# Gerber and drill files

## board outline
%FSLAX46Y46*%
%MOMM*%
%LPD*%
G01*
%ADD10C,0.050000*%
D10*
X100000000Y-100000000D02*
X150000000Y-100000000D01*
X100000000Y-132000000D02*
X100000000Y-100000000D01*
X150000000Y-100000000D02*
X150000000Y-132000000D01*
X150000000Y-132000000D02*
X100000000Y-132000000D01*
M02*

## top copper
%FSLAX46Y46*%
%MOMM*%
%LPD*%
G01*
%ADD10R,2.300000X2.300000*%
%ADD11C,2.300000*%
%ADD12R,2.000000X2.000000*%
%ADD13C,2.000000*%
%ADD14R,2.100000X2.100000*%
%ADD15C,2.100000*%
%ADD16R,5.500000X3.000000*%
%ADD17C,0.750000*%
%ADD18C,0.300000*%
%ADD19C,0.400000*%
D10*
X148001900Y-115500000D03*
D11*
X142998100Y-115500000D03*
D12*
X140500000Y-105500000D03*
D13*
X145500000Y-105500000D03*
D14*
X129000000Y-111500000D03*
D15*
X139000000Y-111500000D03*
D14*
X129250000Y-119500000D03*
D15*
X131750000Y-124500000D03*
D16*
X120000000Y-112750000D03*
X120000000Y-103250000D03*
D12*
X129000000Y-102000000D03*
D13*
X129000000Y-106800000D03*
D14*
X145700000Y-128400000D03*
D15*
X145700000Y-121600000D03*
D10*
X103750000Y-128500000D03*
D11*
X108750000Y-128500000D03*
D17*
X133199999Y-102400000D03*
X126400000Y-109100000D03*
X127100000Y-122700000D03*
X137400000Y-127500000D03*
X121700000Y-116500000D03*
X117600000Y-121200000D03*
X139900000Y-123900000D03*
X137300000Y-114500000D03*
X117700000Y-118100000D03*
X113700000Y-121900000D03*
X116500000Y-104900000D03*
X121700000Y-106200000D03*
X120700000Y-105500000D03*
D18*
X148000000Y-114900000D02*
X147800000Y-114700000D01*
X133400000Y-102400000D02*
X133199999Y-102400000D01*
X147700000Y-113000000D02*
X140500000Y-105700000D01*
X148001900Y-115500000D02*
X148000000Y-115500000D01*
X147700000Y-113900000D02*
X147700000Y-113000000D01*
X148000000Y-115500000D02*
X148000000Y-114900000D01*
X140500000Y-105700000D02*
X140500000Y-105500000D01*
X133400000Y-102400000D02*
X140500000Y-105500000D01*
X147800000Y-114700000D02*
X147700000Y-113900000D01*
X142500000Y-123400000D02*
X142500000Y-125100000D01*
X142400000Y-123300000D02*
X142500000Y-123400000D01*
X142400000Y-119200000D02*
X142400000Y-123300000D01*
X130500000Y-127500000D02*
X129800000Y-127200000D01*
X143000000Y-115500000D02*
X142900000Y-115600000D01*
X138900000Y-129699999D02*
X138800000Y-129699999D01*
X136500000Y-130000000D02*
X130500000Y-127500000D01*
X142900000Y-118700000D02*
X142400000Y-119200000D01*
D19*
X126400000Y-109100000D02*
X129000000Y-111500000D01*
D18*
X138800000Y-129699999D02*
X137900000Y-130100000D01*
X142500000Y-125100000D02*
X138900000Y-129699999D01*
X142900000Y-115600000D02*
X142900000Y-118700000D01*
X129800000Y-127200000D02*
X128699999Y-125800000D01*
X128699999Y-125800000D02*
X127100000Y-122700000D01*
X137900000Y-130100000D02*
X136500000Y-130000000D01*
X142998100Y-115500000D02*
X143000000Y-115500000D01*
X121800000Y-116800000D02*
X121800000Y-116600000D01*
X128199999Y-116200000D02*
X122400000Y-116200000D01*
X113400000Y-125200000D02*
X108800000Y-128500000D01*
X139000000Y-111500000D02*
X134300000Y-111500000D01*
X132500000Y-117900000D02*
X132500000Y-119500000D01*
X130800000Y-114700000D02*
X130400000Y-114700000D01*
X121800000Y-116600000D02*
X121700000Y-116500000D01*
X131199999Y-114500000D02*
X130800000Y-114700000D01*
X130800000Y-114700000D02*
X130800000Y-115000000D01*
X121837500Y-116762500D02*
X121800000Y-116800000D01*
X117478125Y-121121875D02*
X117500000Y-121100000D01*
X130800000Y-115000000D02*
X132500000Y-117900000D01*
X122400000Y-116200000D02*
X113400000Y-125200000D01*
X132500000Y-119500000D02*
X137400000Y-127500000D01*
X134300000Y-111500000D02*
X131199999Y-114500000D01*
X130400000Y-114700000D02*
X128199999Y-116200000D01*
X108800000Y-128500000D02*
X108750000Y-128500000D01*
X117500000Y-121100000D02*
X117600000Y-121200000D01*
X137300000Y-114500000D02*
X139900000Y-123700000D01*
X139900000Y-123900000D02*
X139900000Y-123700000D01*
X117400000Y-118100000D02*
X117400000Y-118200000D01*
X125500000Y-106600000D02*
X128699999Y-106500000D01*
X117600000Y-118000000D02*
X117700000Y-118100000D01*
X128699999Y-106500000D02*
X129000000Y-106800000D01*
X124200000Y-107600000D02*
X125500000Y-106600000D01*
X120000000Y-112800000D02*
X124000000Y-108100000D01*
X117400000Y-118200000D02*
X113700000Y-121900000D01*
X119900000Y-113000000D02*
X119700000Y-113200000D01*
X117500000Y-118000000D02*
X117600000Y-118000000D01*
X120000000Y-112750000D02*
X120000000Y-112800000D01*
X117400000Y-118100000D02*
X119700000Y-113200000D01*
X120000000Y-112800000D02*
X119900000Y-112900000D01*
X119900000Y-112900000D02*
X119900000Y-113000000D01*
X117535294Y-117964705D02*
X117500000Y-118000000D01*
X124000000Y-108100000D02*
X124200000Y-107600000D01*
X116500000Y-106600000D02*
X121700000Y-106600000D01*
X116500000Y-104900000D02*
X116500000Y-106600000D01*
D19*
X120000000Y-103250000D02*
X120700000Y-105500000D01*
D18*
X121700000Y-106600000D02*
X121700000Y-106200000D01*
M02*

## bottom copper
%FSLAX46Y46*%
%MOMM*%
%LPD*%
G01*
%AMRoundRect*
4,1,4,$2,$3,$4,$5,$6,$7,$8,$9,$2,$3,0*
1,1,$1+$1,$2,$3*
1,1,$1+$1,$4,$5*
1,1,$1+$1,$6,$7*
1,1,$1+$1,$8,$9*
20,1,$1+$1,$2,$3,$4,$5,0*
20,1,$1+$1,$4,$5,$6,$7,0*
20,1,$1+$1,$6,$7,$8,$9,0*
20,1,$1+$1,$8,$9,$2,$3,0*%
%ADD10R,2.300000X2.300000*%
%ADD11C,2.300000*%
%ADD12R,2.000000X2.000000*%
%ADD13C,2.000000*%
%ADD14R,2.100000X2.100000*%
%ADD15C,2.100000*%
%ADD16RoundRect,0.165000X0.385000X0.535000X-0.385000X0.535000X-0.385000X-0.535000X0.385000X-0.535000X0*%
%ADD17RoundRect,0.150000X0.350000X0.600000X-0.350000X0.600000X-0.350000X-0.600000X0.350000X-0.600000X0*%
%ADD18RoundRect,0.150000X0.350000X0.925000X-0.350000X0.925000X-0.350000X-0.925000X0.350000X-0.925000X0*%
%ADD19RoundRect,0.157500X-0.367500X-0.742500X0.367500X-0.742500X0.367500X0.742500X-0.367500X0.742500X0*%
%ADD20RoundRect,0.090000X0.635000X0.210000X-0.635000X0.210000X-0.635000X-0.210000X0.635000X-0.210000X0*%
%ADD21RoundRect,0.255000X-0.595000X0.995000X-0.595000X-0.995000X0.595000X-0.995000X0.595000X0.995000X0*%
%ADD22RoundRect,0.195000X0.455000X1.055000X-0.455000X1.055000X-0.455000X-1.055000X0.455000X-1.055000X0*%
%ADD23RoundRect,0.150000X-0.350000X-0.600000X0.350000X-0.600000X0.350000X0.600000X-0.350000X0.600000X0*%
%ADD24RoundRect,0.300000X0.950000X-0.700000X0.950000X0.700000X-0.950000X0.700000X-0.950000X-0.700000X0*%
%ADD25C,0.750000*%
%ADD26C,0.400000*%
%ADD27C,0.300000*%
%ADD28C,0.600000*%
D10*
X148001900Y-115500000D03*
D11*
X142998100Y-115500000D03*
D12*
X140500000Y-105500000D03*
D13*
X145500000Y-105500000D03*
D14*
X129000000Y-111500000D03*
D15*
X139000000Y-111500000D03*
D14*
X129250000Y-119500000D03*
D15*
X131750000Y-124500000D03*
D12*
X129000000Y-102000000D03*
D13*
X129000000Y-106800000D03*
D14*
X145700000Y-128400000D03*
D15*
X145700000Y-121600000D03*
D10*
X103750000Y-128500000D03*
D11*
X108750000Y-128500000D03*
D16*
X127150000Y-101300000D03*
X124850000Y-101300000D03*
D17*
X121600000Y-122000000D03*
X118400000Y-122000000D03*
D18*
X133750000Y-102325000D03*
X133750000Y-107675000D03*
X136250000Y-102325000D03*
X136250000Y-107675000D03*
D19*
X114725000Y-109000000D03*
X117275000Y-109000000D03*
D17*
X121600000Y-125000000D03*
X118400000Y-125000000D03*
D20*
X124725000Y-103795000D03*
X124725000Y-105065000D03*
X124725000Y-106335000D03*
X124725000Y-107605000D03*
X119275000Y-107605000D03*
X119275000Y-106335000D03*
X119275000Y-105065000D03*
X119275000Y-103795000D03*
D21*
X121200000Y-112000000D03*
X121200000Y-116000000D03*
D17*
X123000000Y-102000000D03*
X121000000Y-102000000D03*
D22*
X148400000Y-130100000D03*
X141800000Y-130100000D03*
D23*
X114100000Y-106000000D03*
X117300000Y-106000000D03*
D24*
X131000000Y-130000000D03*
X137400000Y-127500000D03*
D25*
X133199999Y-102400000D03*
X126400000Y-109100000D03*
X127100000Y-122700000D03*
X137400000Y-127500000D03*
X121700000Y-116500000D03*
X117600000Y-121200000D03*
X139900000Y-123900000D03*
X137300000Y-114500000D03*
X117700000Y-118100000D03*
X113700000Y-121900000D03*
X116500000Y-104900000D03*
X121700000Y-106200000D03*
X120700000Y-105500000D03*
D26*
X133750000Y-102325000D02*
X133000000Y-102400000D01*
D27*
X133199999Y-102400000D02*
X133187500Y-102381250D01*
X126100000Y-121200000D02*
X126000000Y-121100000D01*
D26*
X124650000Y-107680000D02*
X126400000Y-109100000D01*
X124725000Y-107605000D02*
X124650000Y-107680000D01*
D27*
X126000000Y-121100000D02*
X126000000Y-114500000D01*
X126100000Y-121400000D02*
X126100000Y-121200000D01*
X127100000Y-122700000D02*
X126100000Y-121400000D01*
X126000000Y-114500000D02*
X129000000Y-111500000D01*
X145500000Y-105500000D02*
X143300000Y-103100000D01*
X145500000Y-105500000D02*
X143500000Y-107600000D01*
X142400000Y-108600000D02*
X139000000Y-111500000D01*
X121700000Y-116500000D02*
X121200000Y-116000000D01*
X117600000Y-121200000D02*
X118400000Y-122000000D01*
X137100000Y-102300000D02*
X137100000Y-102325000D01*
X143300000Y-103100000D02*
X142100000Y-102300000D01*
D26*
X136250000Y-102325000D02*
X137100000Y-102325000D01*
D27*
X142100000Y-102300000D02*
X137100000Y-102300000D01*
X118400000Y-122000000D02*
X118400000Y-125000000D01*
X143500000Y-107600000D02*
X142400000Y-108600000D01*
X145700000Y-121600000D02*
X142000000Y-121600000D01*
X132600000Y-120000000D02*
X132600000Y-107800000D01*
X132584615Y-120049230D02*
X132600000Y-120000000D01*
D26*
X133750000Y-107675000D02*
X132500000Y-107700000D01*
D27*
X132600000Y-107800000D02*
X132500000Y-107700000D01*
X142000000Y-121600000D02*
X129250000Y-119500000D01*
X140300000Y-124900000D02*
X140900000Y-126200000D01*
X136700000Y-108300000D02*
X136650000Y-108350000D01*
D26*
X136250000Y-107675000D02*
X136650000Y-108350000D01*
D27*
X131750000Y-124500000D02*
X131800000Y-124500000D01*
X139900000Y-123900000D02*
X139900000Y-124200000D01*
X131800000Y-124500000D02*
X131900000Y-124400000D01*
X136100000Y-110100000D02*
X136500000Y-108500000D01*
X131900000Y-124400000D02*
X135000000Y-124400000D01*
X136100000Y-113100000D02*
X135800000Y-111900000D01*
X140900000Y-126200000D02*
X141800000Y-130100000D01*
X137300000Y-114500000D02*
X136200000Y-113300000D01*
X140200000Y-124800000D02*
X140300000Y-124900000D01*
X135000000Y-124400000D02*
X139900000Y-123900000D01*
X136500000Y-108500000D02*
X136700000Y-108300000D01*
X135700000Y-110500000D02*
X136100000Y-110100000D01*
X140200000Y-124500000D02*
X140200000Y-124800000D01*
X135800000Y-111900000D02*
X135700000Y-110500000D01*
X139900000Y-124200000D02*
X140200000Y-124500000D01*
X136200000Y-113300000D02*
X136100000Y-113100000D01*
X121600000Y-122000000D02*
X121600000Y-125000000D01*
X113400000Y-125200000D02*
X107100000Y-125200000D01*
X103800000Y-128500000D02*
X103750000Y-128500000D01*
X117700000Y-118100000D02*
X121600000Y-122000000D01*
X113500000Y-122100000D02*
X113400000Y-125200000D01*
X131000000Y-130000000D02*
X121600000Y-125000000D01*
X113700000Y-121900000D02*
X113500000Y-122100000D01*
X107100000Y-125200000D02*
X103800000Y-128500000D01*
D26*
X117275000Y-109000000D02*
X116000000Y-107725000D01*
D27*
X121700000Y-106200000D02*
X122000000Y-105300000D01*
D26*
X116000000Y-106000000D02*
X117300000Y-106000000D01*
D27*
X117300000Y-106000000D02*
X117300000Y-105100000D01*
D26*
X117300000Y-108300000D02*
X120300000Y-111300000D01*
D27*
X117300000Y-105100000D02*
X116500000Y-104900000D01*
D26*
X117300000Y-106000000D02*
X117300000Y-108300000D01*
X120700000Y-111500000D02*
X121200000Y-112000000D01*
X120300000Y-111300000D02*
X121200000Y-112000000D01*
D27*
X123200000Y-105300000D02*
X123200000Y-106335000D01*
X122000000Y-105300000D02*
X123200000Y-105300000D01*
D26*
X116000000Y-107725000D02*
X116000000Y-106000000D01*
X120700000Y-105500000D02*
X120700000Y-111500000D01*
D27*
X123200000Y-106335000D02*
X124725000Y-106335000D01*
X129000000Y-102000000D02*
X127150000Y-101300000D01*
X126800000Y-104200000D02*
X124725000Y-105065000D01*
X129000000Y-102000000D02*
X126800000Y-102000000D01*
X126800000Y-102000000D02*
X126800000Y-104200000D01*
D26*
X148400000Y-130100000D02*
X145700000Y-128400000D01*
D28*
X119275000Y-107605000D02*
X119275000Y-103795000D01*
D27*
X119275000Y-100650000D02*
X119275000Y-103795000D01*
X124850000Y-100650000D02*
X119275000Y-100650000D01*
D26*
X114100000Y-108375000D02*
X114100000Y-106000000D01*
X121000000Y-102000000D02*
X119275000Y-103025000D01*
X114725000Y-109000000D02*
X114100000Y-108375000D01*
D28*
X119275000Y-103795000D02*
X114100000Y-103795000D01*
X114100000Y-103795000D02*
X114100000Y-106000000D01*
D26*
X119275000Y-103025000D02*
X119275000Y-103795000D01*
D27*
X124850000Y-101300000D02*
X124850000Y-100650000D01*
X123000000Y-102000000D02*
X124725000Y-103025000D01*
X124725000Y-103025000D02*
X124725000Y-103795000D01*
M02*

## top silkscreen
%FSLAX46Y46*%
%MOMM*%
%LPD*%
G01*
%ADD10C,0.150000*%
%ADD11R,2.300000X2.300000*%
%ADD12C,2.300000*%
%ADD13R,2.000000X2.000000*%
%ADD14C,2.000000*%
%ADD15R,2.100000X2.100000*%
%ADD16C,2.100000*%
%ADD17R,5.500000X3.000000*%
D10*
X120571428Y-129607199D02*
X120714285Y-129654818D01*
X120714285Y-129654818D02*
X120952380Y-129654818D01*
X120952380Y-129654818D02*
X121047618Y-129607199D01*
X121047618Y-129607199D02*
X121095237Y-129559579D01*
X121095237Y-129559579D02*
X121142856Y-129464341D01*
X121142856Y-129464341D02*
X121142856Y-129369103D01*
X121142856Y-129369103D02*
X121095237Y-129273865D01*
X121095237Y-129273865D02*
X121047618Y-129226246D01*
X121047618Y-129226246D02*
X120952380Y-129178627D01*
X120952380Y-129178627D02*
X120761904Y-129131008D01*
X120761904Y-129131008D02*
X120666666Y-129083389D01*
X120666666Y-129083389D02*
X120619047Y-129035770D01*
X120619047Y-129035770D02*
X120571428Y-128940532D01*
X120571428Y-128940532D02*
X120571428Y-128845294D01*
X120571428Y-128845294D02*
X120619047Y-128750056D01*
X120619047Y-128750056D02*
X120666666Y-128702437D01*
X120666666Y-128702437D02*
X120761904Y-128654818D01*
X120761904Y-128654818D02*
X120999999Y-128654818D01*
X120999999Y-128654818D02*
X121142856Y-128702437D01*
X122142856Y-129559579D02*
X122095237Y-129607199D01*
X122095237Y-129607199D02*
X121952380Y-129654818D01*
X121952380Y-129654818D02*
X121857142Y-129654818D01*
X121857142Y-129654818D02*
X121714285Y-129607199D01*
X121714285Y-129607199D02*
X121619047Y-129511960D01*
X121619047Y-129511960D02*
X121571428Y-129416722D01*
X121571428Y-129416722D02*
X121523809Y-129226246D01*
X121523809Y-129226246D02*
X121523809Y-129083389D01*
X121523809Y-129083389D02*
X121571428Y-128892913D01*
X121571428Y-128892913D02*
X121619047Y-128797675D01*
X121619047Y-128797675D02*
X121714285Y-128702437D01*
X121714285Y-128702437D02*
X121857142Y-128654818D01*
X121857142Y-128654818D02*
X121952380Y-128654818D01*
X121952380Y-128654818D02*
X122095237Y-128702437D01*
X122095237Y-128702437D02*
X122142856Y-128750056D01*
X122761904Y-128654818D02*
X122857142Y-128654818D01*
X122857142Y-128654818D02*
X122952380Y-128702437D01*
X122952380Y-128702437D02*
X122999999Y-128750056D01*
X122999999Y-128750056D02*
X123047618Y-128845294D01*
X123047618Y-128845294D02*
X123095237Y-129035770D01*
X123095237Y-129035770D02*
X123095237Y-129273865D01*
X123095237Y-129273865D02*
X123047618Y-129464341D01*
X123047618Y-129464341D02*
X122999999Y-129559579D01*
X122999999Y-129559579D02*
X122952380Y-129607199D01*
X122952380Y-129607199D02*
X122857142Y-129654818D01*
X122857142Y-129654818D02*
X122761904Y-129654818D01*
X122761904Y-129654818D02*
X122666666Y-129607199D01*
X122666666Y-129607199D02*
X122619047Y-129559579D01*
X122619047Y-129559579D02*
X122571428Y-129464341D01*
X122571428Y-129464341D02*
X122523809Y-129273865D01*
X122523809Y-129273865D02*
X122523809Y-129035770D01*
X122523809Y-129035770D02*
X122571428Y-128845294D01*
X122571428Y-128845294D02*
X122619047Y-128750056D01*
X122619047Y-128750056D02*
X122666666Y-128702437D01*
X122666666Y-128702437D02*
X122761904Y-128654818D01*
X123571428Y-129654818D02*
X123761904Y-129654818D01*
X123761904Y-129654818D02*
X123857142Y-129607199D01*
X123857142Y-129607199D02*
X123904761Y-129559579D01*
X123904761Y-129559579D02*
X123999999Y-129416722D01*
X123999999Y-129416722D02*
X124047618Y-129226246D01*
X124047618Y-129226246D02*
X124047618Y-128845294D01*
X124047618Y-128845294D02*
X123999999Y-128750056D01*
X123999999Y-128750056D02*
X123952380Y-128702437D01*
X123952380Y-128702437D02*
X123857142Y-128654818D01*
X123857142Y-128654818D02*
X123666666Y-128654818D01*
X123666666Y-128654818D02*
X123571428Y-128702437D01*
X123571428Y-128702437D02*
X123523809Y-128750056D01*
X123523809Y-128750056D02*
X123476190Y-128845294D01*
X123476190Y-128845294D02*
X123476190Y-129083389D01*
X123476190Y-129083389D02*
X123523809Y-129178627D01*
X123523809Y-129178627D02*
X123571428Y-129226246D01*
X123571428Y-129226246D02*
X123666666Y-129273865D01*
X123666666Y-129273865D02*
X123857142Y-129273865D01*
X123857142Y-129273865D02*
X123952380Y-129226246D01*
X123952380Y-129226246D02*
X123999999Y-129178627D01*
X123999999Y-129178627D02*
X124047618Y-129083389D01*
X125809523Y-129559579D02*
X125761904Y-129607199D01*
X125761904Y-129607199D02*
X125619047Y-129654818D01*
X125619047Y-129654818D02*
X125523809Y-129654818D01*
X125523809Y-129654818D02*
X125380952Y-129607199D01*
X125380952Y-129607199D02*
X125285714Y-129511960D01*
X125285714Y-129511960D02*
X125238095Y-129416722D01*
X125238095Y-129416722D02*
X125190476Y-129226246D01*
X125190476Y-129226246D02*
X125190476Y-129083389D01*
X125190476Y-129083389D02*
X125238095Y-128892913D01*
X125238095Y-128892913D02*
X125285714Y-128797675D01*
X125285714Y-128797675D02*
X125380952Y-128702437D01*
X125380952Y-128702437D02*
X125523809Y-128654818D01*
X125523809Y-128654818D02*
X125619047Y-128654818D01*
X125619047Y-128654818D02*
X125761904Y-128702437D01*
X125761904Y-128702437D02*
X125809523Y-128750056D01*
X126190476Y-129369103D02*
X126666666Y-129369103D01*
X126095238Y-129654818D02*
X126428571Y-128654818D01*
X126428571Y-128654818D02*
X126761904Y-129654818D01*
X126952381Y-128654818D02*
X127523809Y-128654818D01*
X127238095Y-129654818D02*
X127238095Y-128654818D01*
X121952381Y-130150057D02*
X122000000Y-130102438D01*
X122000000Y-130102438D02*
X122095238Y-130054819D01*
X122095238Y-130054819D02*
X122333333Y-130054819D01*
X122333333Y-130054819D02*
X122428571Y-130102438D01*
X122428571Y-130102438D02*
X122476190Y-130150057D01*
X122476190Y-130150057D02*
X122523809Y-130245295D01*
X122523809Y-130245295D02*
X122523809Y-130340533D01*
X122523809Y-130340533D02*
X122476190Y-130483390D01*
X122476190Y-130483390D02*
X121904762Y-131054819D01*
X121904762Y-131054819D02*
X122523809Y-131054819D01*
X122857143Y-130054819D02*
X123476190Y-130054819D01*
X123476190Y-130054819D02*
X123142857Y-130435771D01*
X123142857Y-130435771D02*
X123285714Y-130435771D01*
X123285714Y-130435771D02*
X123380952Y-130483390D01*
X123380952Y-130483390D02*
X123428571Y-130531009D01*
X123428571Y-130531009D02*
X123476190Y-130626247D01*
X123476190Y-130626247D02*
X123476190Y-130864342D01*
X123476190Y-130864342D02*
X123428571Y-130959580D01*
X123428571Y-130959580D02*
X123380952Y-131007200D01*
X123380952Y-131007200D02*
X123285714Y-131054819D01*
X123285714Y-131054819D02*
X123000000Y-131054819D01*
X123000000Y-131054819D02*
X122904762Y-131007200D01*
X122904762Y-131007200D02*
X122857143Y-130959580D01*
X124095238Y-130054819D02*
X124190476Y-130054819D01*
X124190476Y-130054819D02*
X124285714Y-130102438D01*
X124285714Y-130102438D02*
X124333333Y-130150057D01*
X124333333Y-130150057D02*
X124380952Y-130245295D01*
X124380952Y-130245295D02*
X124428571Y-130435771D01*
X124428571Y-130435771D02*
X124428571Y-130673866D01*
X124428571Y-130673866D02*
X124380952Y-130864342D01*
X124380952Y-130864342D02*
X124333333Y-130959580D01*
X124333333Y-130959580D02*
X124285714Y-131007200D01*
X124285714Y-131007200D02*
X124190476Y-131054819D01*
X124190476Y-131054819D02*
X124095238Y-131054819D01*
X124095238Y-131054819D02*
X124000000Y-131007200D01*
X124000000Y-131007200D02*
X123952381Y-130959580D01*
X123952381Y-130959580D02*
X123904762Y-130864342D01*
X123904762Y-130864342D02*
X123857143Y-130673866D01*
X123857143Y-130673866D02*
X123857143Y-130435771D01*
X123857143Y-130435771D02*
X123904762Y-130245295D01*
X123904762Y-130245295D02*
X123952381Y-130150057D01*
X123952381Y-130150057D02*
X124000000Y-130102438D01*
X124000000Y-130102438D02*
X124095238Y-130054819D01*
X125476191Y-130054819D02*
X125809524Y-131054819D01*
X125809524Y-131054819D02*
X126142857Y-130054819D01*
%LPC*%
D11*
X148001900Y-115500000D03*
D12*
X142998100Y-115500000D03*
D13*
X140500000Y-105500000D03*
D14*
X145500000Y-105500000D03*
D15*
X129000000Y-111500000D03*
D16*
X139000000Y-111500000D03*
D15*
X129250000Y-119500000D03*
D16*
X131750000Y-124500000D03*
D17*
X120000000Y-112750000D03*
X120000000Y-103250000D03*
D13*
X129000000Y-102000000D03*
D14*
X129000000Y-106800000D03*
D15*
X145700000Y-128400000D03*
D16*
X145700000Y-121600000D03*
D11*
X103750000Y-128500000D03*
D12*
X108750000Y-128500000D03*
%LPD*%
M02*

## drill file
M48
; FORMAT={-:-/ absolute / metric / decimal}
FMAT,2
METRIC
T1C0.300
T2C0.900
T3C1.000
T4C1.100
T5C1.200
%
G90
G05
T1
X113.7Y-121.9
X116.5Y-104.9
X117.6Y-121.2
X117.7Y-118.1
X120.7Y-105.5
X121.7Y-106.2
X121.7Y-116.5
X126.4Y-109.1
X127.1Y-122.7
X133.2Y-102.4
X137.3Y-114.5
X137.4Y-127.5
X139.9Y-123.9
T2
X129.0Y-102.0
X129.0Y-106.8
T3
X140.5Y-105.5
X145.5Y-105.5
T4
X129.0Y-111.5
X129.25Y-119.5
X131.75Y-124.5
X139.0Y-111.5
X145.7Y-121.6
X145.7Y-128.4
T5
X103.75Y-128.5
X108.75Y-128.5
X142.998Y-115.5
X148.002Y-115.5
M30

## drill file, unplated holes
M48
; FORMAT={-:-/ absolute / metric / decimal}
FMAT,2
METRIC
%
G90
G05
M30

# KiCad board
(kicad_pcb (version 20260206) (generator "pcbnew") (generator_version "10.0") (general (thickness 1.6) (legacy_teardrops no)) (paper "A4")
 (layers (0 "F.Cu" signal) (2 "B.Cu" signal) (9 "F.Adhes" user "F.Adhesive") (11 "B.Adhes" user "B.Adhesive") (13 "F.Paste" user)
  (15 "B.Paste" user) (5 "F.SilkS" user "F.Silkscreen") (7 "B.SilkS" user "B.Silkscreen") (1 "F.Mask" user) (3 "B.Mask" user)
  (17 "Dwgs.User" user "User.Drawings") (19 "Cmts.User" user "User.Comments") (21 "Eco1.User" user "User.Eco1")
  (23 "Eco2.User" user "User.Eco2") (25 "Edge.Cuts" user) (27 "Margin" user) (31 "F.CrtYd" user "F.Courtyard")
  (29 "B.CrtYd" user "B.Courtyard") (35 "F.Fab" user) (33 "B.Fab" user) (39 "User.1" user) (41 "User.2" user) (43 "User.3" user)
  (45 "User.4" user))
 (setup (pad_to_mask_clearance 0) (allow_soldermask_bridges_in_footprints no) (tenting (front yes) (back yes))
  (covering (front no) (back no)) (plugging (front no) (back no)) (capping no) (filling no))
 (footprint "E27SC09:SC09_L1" (layer "F.Cu") (at 145.5 115.5 180)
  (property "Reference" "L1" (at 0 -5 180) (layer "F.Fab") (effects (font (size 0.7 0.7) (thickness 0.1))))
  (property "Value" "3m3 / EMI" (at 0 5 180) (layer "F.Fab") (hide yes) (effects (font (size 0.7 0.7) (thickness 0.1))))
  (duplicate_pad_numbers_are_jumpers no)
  (pad "1" thru_hole rect (at -2.5019 0 180) (size 2.3 2.3) (drill 1.2) (layers "*.Cu" "*.Mask") (remove_unused_layers no) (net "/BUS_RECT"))
  (pad "2" thru_hole circle (at 2.5019 0 180) (size 2.3 2.3) (drill 1.2) (layers "*.Cu" "*.Mask") (remove_unused_layers no)
   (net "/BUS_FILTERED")))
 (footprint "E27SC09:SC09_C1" (layer "F.Cu") (at 143 105.5)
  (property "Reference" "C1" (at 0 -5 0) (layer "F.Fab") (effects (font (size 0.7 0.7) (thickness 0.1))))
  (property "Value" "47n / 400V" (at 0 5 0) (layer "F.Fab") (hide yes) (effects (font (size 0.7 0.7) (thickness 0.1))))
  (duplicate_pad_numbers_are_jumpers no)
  (pad "1" thru_hole rect (at -2.5 0) (size 2 2) (drill 1) (layers "*.Cu" "*.Mask") (remove_unused_layers no) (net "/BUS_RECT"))
  (pad "2" thru_hole circle (at 2.5 0) (size 2 2) (drill 1) (layers "*.Cu" "*.Mask") (remove_unused_layers no) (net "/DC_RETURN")))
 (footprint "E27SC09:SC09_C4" (layer "F.Cu") (at 134 111.5)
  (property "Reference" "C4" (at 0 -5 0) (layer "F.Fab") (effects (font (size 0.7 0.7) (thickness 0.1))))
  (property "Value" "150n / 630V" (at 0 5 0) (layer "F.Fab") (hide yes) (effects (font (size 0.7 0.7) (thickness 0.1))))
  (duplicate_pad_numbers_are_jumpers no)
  (pad "1" thru_hole rect (at -5 0) (size 2.1 2.1) (drill 1.1) (layers "*.Cu" "*.Mask") (remove_unused_layers no) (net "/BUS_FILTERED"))
  (pad "2" thru_hole circle (at 5 0) (size 2.1 2.1) (drill 1.1) (layers "*.Cu" "*.Mask") (remove_unused_layers no) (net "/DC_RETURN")))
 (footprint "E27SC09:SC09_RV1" (layer "F.Cu") (at 130.5 122)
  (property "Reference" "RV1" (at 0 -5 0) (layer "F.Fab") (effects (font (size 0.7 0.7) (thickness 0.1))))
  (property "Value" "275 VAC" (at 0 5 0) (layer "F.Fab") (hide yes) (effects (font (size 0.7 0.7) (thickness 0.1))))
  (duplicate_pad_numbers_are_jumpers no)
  (pad "1" thru_hole rect (at -1.25 -2.5) (size 2.1 2.1) (drill 1.1) (layers "*.Cu" "*.Mask") (remove_unused_layers no) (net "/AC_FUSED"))
  (pad "2" thru_hole circle (at 1.25 2.5) (size 2.1 2.1) (drill 1.1) (layers "*.Cu" "*.Mask") (remove_unused_layers no) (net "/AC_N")))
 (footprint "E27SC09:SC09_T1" (layer "F.Cu") (at 120 108)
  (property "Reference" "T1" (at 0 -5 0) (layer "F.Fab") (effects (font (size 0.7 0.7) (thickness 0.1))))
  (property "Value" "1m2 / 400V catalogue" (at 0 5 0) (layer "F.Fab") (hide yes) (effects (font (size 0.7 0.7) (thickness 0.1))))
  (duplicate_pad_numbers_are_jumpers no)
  (pad "1" smd rect (at 0 4.75) (size 5.5 3) (layers "F.Cu" "F.Mask" "F.Paste") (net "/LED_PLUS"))
  (pad "2" smd rect (at 0 -4.75) (size 5.5 3) (layers "F.Cu" "F.Mask" "F.Paste") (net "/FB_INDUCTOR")))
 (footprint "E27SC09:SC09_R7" (layer "F.Cu") (at 129 102)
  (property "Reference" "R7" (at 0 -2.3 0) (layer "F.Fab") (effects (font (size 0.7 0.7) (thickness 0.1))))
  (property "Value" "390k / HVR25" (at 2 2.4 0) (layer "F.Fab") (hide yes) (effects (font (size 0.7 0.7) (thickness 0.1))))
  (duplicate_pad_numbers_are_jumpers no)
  (pad "1" thru_hole rect (at 0 0) (size 2 2) (drill 0.9) (layers "*.Cu" "*.Mask") (remove_unused_layers no) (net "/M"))
  (pad "2" thru_hole circle (at 0 4.8) (size 2 2) (drill 0.9) (layers "*.Cu" "*.Mask") (remove_unused_layers no) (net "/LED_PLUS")))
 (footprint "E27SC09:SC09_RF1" (layer "F.Cu") (at 145.7 128.4 180)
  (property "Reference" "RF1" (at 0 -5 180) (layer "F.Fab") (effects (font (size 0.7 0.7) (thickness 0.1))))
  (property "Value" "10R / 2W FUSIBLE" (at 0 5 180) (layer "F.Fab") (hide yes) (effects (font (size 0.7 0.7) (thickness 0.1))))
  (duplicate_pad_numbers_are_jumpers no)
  (pad "1" thru_hole rect (at 0 0 180) (size 2.1 2.1) (drill 1.1) (layers "*.Cu" "*.Mask") (remove_unused_layers no) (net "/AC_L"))
  (pad "2" thru_hole circle (at 0 6.8 180) (size 2.1 2.1) (drill 1.1) (layers "*.Cu" "*.Mask") (remove_unused_layers no) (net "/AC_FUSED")))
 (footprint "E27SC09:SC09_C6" (layer "F.Cu") (at 106.25 128.5 90)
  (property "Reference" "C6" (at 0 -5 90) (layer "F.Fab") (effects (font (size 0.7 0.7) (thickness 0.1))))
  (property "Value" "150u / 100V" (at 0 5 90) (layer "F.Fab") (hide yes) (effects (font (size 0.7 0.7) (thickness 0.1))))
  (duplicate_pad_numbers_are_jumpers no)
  (pad "1" thru_hole rect (at 0 -2.5 90) (size 2.3 2.3) (drill 1.2) (layers "*.Cu" "*.Mask") (remove_unused_layers no) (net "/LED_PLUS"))
  (pad "2" thru_hole circle (at 0 2.5 90) (size 2.3 2.3) (drill 1.2) (layers "*.Cu" "*.Mask") (remove_unused_layers no) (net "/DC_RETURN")))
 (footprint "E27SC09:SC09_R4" (layer "B.Cu") (at 126 101.3 180)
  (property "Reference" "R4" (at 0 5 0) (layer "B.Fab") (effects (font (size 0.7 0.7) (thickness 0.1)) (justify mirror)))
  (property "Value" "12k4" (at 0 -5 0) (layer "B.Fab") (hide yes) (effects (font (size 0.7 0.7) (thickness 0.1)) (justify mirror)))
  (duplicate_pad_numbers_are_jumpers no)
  (pad "1" smd roundrect (at -1.15 0 180) (size 1.1 1.4) (layers "B.Cu" "B.Mask" "B.Paste") (roundrect_rratio 0.15) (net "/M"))
  (pad "2" smd roundrect (at 1.15 0 180) (size 1.1 1.4) (layers "B.Cu" "B.Mask" "B.Paste") (roundrect_rratio 0.15) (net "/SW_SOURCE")))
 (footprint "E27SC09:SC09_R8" (layer "B.Cu") (at 120 122 180)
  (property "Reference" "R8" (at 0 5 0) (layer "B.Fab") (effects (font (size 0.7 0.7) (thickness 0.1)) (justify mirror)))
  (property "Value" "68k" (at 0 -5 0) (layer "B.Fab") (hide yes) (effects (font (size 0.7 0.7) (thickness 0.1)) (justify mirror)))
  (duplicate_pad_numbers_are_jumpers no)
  (pad "1" smd roundrect (at -1.6 0 180) (size 1 1.5) (layers "B.Cu" "B.Mask" "B.Paste") (roundrect_rratio 0.15) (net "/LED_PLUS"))
  (pad "2" smd roundrect (at 1.6 0 180) (size 1 1.5) (layers "B.Cu" "B.Mask" "B.Paste") (roundrect_rratio 0.15) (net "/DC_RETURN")))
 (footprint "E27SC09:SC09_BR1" (layer "B.Cu") (at 135 105 180)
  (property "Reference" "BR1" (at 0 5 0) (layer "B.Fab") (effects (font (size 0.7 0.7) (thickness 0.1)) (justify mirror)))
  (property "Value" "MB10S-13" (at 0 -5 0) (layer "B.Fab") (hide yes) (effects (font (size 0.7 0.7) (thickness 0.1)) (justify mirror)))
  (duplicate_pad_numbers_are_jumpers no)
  (pad "1" smd roundrect (at 1.25 2.675 180) (size 1 2.15) (layers "B.Cu" "B.Mask" "B.Paste") (roundrect_rratio 0.15) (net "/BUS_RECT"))
  (pad "2" smd roundrect (at 1.25 -2.675 180) (size 1 2.15) (layers "B.Cu" "B.Mask" "B.Paste") (roundrect_rratio 0.15) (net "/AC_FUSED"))
  (pad "3" smd roundrect (at -1.25 2.675 180) (size 1 2.15) (layers "B.Cu" "B.Mask" "B.Paste") (roundrect_rratio 0.15) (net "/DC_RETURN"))
  (pad "4" smd roundrect (at -1.25 -2.675 180) (size 1 2.15) (layers "B.Cu" "B.Mask" "B.Paste") (roundrect_rratio 0.15) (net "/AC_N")))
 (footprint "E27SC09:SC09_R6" (layer "B.Cu") (at 116 109)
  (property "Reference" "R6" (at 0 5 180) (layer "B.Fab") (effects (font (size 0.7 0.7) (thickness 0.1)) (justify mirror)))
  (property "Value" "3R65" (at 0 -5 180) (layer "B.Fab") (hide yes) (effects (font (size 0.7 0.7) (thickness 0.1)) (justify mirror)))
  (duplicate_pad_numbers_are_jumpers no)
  (pad "1" smd roundrect (at -1.275 0) (size 1.05 1.8) (layers "B.Cu" "B.Mask" "B.Paste") (roundrect_rratio 0.15) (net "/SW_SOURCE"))
  (pad "2" smd roundrect (at 1.275 0) (size 1.05 1.8) (layers "B.Cu" "B.Mask" "B.Paste") (roundrect_rratio 0.15) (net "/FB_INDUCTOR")))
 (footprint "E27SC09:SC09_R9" (layer "B.Cu") (at 120 125 180)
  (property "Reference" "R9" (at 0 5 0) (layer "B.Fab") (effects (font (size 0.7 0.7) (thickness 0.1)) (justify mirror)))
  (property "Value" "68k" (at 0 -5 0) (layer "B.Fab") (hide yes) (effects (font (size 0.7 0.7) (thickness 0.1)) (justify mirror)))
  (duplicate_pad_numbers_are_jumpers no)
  (pad "1" smd roundrect (at -1.6 0 180) (size 1 1.5) (layers "B.Cu" "B.Mask" "B.Paste") (roundrect_rratio 0.15) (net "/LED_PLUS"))
  (pad "2" smd roundrect (at 1.6 0 180) (size 1 1.5) (layers "B.Cu" "B.Mask" "B.Paste") (roundrect_rratio 0.15) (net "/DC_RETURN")))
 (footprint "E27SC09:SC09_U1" (layer "B.Cu") (at 122 105.7 180)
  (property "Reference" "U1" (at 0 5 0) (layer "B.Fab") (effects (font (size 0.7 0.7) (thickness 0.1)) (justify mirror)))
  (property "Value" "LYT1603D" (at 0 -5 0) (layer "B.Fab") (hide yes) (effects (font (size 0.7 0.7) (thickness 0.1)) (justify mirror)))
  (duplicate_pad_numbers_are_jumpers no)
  (pad "1" smd roundrect (at -2.725 1.905 180) (size 1.45 0.6) (layers "B.Cu" "B.Mask" "B.Paste") (roundrect_rratio 0.15) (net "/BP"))
  (pad "2" smd roundrect (at -2.725 0.635 180) (size 1.45 0.6) (layers "B.Cu" "B.Mask" "B.Paste") (roundrect_rratio 0.15) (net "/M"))
  (pad "3" smd roundrect (at -2.725 -0.635 180) (size 1.45 0.6) (layers "B.Cu" "B.Mask" "B.Paste") (roundrect_rratio 0.15)
   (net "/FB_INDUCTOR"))
  (pad "4" smd roundrect (at -2.725 -1.905 180) (size 1.45 0.6) (layers "B.Cu" "B.Mask" "B.Paste") (roundrect_rratio 0.15)
   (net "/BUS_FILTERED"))
  (pad "5" smd roundrect (at 2.725 -1.905 180) (size 1.45 0.6) (layers "B.Cu" "B.Mask" "B.Paste") (roundrect_rratio 0.15) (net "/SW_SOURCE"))
  (pad "6" smd roundrect (at 2.725 -0.635 180) (size 1.45 0.6) (layers "B.Cu" "B.Mask" "B.Paste") (roundrect_rratio 0.15) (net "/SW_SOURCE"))
  (pad "7" smd roundrect (at 2.725 0.635 180) (size 1.45 0.6) (layers "B.Cu" "B.Mask" "B.Paste") (roundrect_rratio 0.15) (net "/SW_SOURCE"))
  (pad "8" smd roundrect (at 2.725 1.905 180) (size 1.45 0.6) (layers "B.Cu" "B.Mask" "B.Paste") (roundrect_rratio 0.15) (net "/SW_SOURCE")))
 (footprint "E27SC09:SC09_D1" (layer "B.Cu") (at 121.2 114 -90)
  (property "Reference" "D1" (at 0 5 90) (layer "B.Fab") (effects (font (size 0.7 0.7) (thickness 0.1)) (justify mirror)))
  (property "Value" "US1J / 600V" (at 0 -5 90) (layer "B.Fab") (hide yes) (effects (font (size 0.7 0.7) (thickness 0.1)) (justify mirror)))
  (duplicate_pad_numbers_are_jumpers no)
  (pad "1" smd roundrect (at -2 0 270) (size 2.5 1.7) (layers "B.Cu" "B.Mask" "B.Paste") (roundrect_rratio 0.15) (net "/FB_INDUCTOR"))
  (pad "2" smd roundrect (at 2 0 270) (size 2.5 1.7) (layers "B.Cu" "B.Mask" "B.Paste") (roundrect_rratio 0.15) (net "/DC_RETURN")))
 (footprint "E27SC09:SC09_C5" (layer "B.Cu") (at 122 102 180)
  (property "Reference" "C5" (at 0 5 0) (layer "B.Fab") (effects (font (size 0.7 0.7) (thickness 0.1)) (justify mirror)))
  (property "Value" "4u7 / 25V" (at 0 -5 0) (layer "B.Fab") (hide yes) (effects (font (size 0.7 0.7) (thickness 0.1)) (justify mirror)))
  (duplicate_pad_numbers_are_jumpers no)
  (pad "1" smd roundrect (at -1 0 180) (size 1 1.5) (layers "B.Cu" "B.Mask" "B.Paste") (roundrect_rratio 0.15) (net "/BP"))
  (pad "2" smd roundrect (at 1 0 180) (size 1 1.5) (layers "B.Cu" "B.Mask" "B.Paste") (roundrect_rratio 0.15) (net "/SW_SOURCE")))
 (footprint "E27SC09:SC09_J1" (layer "B.Cu") (at 148.4 130.1 180)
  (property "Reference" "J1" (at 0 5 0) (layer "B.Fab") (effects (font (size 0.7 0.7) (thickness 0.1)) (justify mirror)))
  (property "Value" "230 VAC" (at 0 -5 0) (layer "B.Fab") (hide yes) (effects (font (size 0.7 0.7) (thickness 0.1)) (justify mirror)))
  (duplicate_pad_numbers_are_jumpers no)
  (pad "1" smd roundrect (at 0 0 180) (size 1.3 2.5) (layers "B.Cu" "B.Mask" "B.Paste") (roundrect_rratio 0.15) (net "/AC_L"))
  (pad "2" smd roundrect (at 6.6 0 180) (size 1.3 2.5) (layers "B.Cu" "B.Mask" "B.Paste") (roundrect_rratio 0.15) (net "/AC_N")))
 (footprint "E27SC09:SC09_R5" (layer "B.Cu") (at 115.7 106)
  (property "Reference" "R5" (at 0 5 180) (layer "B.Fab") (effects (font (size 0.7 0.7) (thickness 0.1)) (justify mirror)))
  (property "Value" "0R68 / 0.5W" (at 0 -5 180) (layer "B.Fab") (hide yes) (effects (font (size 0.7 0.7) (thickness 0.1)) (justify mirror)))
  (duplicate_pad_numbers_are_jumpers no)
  (pad "1" smd roundrect (at -1.6 0) (size 1 1.5) (layers "B.Cu" "B.Mask" "B.Paste") (roundrect_rratio 0.15) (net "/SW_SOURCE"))
  (pad "2" smd roundrect (at 1.6 0) (size 1 1.5) (layers "B.Cu" "B.Mask" "B.Paste") (roundrect_rratio 0.15) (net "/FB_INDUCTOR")))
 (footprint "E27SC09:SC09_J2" (layer "B.Cu") (at 131 130 90)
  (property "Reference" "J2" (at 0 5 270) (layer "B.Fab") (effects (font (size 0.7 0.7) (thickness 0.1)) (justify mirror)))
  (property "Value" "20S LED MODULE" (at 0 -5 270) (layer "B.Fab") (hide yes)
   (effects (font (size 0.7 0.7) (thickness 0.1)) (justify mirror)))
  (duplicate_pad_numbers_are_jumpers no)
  (pad "1" smd roundrect (at 0 0 90) (size 2 2.5) (layers "B.Cu" "B.Mask" "B.Paste") (roundrect_rratio 0.15) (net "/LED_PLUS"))
  (pad "2" smd roundrect (at 2.5 6.4 90) (size 2 2.5) (layers "B.Cu" "B.Mask" "B.Paste") (roundrect_rratio 0.15) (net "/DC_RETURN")))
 (gr_line (start 100 100) (end 150 100) (stroke (width 0.05) (type default)) (layer "Edge.Cuts"))
 (gr_line (start 100 132) (end 100 100) (stroke (width 0.05) (type default)) (layer "Edge.Cuts"))
 (gr_line (start 150 100) (end 150 132) (stroke (width 0.05) (type default)) (layer "Edge.Cuts"))
 (gr_line (start 150 132) (end 100 132) (stroke (width 0.05) (type default)) (layer "Edge.Cuts"))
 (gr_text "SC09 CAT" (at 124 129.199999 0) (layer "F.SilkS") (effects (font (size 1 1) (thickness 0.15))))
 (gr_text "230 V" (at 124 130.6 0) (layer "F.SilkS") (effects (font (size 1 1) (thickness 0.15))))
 (segment (start 148 114.9) (end 147.8 114.7) (width 0.3) (layer "F.Cu") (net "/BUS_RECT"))
 (segment (start 133.4 102.4) (end 133.199999 102.4) (width 0.3) (layer "F.Cu") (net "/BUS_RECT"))
 (segment (start 147.7 113) (end 140.5 105.7) (width 0.3) (layer "F.Cu") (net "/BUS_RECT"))
 (segment (start 148.0019 115.5) (end 148 115.5) (width 0.3) (layer "F.Cu") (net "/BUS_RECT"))
 (segment (start 147.7 113.9) (end 147.7 113) (width 0.3) (layer "F.Cu") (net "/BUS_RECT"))
 (segment (start 148 115.5) (end 148 114.9) (width 0.3) (layer "F.Cu") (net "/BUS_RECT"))
 (segment (start 140.5 105.7) (end 140.5 105.5) (width 0.3) (layer "F.Cu") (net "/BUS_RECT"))
 (segment (start 133.4 102.4) (end 140.5 105.5) (width 0.3) (layer "F.Cu") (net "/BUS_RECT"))
 (segment (start 147.8 114.7) (end 147.7 113.9) (width 0.3) (layer "F.Cu") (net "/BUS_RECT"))
 (via (at 133.199999 102.4) (size 0.75) (drill 0.3) (layers "F.Cu" "B.Cu") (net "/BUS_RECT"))
 (segment (start 133.75 102.325) (end 133 102.4) (width 0.4) (layer "B.Cu") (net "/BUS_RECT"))
 (segment (start 133.199999 102.4) (end 133.1875 102.38125) (width 0.3) (layer "B.Cu") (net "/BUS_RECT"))
 (segment (start 142.5 123.4) (end 142.5 125.1) (width 0.3) (layer "F.Cu") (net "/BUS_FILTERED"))
 (segment (start 142.4 123.3) (end 142.5 123.4) (width 0.3) (layer "F.Cu") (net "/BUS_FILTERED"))
 (segment (start 142.4 119.2) (end 142.4 123.3) (width 0.3) (layer "F.Cu") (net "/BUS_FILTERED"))
 (segment (start 130.5 127.5) (end 129.8 127.2) (width 0.3) (layer "F.Cu") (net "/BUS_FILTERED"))
 (segment (start 143 115.5) (end 142.9 115.6) (width 0.3) (layer "F.Cu") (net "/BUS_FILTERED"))
 (segment (start 138.9 129.699999) (end 138.8 129.699999) (width 0.3) (layer "F.Cu") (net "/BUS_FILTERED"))
 (segment (start 136.5 130) (end 130.5 127.5) (width 0.3) (layer "F.Cu") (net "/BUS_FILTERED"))
 (segment (start 142.9 118.7) (end 142.4 119.2) (width 0.3) (layer "F.Cu") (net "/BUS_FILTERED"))
 (segment (start 126.4 109.1) (end 129 111.5) (width 0.4) (layer "F.Cu") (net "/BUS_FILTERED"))
 (segment (start 138.8 129.699999) (end 137.9 130.1) (width 0.3) (layer "F.Cu") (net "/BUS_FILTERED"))
 (segment (start 142.5 125.1) (end 138.9 129.699999) (width 0.3) (layer "F.Cu") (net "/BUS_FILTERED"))
 (segment (start 142.9 115.6) (end 142.9 118.7) (width 0.3) (layer "F.Cu") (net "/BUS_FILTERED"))
 (segment (start 129.8 127.2) (end 128.699999 125.8) (width 0.3) (layer "F.Cu") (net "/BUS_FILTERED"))
 (segment (start 128.699999 125.8) (end 127.1 122.7) (width 0.3) (layer "F.Cu") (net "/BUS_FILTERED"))
 (segment (start 137.9 130.1) (end 136.5 130) (width 0.3) (layer "F.Cu") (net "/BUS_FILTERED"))
 (segment (start 142.9981 115.5) (end 143 115.5) (width 0.3) (layer "F.Cu") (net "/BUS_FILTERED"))
 (via (at 126.4 109.1) (size 0.75) (drill 0.3) (layers "F.Cu" "B.Cu") (tenting (front yes) (back yes)) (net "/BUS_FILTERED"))
 (via (at 127.1 122.7) (size 0.75) (drill 0.3) (layers "F.Cu" "B.Cu") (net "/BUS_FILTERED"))
 (segment (start 126.1 121.2) (end 126 121.1) (width 0.3) (layer "B.Cu") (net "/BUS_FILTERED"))
 (segment (start 124.65 107.68) (end 126.4 109.1) (width 0.4) (layer "B.Cu") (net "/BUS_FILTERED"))
 (segment (start 124.725 107.605) (end 124.65 107.68) (width 0.4) (layer "B.Cu") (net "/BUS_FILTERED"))
 (segment (start 126 121.1) (end 126 114.5) (width 0.3) (layer "B.Cu") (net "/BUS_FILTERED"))
 (segment (start 126.1 121.4) (end 126.1 121.2) (width 0.3) (layer "B.Cu") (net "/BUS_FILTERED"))
 (segment (start 127.1 122.7) (end 126.1 121.4) (width 0.3) (layer "B.Cu") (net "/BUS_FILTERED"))
 (segment (start 126 114.5) (end 129 111.5) (width 0.3) (layer "B.Cu") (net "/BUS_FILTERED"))
 (segment (start 121.8 116.8) (end 121.8 116.6) (width 0.3) (layer "F.Cu") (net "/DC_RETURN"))
 (segment (start 128.199999 116.2) (end 122.4 116.2) (width 0.3) (layer "F.Cu") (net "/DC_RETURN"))
 (segment (start 113.4 125.2) (end 108.8 128.5) (width 0.3) (layer "F.Cu") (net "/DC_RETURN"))
 (segment (start 139 111.5) (end 134.3 111.5) (width 0.3) (layer "F.Cu") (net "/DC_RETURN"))
 (segment (start 132.5 117.9) (end 132.5 119.5) (width 0.3) (layer "F.Cu") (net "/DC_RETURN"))
 (segment (start 130.8 114.7) (end 130.4 114.7) (width 0.3) (layer "F.Cu") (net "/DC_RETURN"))
 (segment (start 121.8 116.6) (end 121.7 116.5) (width 0.3) (layer "F.Cu") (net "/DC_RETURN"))
 (segment (start 131.199999 114.5) (end 130.8 114.7) (width 0.3) (layer "F.Cu") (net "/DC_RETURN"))
 (segment (start 130.8 114.7) (end 130.8 115) (width 0.3) (layer "F.Cu") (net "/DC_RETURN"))
 (segment (start 121.8375 116.7625) (end 121.8 116.8) (width 0.3) (layer "F.Cu") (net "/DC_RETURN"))
 (segment (start 117.478125 121.121875) (end 117.5 121.1) (width 0.3) (layer "F.Cu") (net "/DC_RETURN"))
 (segment (start 130.8 115) (end 132.5 117.9) (width 0.3) (layer "F.Cu") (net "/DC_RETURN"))
 (segment (start 122.4 116.2) (end 113.4 125.2) (width 0.3) (layer "F.Cu") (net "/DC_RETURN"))
 (segment (start 132.5 119.5) (end 137.4 127.5) (width 0.3) (layer "F.Cu") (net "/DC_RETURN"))
 (segment (start 134.3 111.5) (end 131.199999 114.5) (width 0.3) (layer "F.Cu") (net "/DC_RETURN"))
 (segment (start 130.4 114.7) (end 128.199999 116.2) (width 0.3) (layer "F.Cu") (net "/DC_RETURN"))
 (segment (start 108.8 128.5) (end 108.75 128.5) (width 0.3) (layer "F.Cu") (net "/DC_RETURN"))
 (segment (start 117.5 121.1) (end 117.6 121.2) (width 0.3) (layer "F.Cu") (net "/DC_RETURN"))
 (via (at 137.4 127.5) (size 0.75) (drill 0.3) (layers "F.Cu" "B.Cu") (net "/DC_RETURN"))
 (via (at 121.7 116.5) (size 0.75) (drill 0.3) (layers "F.Cu" "B.Cu") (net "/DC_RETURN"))
 (via (at 117.6 121.2) (size 0.75) (drill 0.3) (layers "F.Cu" "B.Cu") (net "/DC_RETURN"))
 (segment (start 145.5 105.5) (end 143.3 103.1) (width 0.3) (layer "B.Cu") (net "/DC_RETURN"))
 (segment (start 145.5 105.5) (end 143.5 107.6) (width 0.3) (layer "B.Cu") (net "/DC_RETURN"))
 (segment (start 142.4 108.6) (end 139 111.5) (width 0.3) (layer "B.Cu") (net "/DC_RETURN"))
 (segment (start 121.7 116.5) (end 121.2 116) (width 0.3) (layer "B.Cu") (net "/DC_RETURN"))
 (segment (start 117.6 121.2) (end 118.4 122) (width 0.3) (layer "B.Cu") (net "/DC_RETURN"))
 (segment (start 137.1 102.3) (end 137.1 102.325) (width 0.3) (layer "B.Cu") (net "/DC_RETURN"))
 (segment (start 143.3 103.1) (end 142.1 102.3) (width 0.3) (layer "B.Cu") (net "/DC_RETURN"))
 (segment (start 136.25 102.325) (end 137.1 102.325) (width 0.4) (layer "B.Cu") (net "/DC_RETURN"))
 (segment (start 142.1 102.3) (end 137.1 102.3) (width 0.3) (layer "B.Cu") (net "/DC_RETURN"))
 (segment (start 118.4 122) (end 118.4 125) (width 0.3) (layer "B.Cu") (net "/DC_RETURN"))
 (segment (start 143.5 107.6) (end 142.4 108.6) (width 0.3) (layer "B.Cu") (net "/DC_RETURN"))
 (segment (start 145.7 121.6) (end 142 121.6) (width 0.3) (layer "B.Cu") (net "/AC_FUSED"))
 (segment (start 132.6 120) (end 132.6 107.8) (width 0.3) (layer "B.Cu") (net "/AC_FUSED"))
 (segment (start 132.584615 120.04923) (end 132.6 120) (width 0.3) (layer "B.Cu") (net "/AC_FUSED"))
 (segment (start 133.75 107.675) (end 132.5 107.7) (width 0.4) (layer "B.Cu") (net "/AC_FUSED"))
 (segment (start 132.6 107.8) (end 132.5 107.7) (width 0.3) (layer "B.Cu") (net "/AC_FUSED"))
 (segment (start 142 121.6) (end 129.25 119.5) (width 0.3) (layer "B.Cu") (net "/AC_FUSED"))
 (segment (start 137.3 114.5) (end 139.9 123.7) (width 0.3) (layer "F.Cu") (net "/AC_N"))
 (segment (start 139.9 123.9) (end 139.9 123.7) (width 0.3) (layer "F.Cu") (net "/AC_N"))
 (via (at 139.9 123.9) (size 0.75) (drill 0.3) (layers "F.Cu" "B.Cu") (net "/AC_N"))
 (via (at 137.3 114.5) (size 0.75) (drill 0.3) (layers "F.Cu" "B.Cu") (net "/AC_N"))
 (segment (start 140.3 124.9) (end 140.9 126.2) (width 0.3) (layer "B.Cu") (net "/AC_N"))
 (segment (start 136.7 108.3) (end 136.65 108.35) (width 0.3) (layer "B.Cu") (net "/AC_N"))
 (segment (start 136.25 107.675) (end 136.65 108.35) (width 0.4) (layer "B.Cu") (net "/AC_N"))
 (segment (start 131.75 124.5) (end 131.8 124.5) (width 0.3) (layer "B.Cu") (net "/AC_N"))
 (segment (start 139.9 123.9) (end 139.9 124.2) (width 0.3) (layer "B.Cu") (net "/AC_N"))
 (segment (start 131.8 124.5) (end 131.9 124.4) (width 0.3) (layer "B.Cu") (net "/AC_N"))
 (segment (start 136.1 110.1) (end 136.5 108.5) (width 0.3) (layer "B.Cu") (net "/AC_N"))
 (segment (start 131.9 124.4) (end 135 124.4) (width 0.3) (layer "B.Cu") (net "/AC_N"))
 (segment (start 136.1 113.1) (end 135.8 111.9) (width 0.3) (layer "B.Cu") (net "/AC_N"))
 (segment (start 140.9 126.2) (end 141.8 130.1) (width 0.3) (layer "B.Cu") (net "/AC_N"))
 (segment (start 137.3 114.5) (end 136.2 113.3) (width 0.3) (layer "B.Cu") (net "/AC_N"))
 (segment (start 140.2 124.8) (end 140.3 124.9) (width 0.3) (layer "B.Cu") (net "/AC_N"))
 (segment (start 135 124.4) (end 139.9 123.9) (width 0.3) (layer "B.Cu") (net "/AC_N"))
 (segment (start 136.5 108.5) (end 136.7 108.3) (width 0.3) (layer "B.Cu") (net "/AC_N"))
 (segment (start 135.7 110.5) (end 136.1 110.1) (width 0.3) (layer "B.Cu") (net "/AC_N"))
 (segment (start 140.2 124.5) (end 140.2 124.8) (width 0.3) (layer "B.Cu") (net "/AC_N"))
 (segment (start 135.8 111.9) (end 135.7 110.5) (width 0.3) (layer "B.Cu") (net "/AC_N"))
 (segment (start 139.9 124.2) (end 140.2 124.5) (width 0.3) (layer "B.Cu") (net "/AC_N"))
 (segment (start 136.2 113.3) (end 136.1 113.1) (width 0.3) (layer "B.Cu") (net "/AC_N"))
 (segment (start 117.4 118.1) (end 117.4 118.2) (width 0.3) (layer "F.Cu") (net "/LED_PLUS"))
 (segment (start 125.5 106.6) (end 128.699999 106.5) (width 0.3) (layer "F.Cu") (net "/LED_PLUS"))
 (segment (start 117.6 118) (end 117.7 118.1) (width 0.3) (layer "F.Cu") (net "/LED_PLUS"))
 (segment (start 128.699999 106.5) (end 129 106.8) (width 0.3) (layer "F.Cu") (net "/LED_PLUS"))
 (segment (start 124.2 107.6) (end 125.5 106.6) (width 0.3) (layer "F.Cu") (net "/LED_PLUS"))
 (segment (start 120 112.8) (end 124 108.1) (width 0.3) (layer "F.Cu") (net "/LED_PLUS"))
 (segment (start 117.4 118.2) (end 113.7 121.9) (width 0.3) (layer "F.Cu") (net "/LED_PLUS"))
 (segment (start 119.9 113) (end 119.7 113.2) (width 0.3) (layer "F.Cu") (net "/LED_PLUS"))
 (segment (start 117.5 118) (end 117.6 118) (width 0.3) (layer "F.Cu") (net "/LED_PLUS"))
 (segment (start 120 112.75) (end 120 112.8) (width 0.3) (layer "F.Cu") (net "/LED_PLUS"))
 (segment (start 117.4 118.1) (end 119.7 113.2) (width 0.3) (layer "F.Cu") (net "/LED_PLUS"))
 (segment (start 120 112.8) (end 119.9 112.9) (width 0.3) (layer "F.Cu") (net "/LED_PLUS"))
 (segment (start 119.9 112.9) (end 119.9 113) (width 0.3) (layer "F.Cu") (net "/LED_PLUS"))
 (segment (start 117.535294 117.964705) (end 117.5 118) (width 0.3) (layer "F.Cu") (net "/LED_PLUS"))
 (segment (start 124 108.1) (end 124.2 107.6) (width 0.3) (layer "F.Cu") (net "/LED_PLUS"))
 (via (at 117.7 118.1) (size 0.75) (drill 0.3) (layers "F.Cu" "B.Cu") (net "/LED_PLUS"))
 (via (at 113.7 121.9) (size 0.75) (drill 0.3) (layers "F.Cu" "B.Cu") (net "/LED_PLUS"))
 (segment (start 121.6 122) (end 121.6 125) (width 0.3) (layer "B.Cu") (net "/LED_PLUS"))
 (segment (start 113.4 125.2) (end 107.1 125.2) (width 0.3) (layer "B.Cu") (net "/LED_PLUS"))
 (segment (start 103.8 128.5) (end 103.75 128.5) (width 0.3) (layer "B.Cu") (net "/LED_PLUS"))
 (segment (start 117.7 118.1) (end 121.6 122) (width 0.3) (layer "B.Cu") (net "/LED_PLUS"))
 (segment (start 113.5 122.1) (end 113.4 125.2) (width 0.3) (layer "B.Cu") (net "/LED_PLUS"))
 (segment (start 131 130) (end 121.6 125) (width 0.3) (layer "B.Cu") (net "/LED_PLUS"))
 (segment (start 113.7 121.9) (end 113.5 122.1) (width 0.3) (layer "B.Cu") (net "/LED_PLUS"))
 (segment (start 107.1 125.2) (end 103.8 128.5) (width 0.3) (layer "B.Cu") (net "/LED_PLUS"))
 (segment (start 116.5 106.6) (end 121.7 106.6) (width 0.3) (layer "F.Cu") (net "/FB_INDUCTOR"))
 (segment (start 116.5 104.9) (end 116.5 106.6) (width 0.3) (layer "F.Cu") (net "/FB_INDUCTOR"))
 (segment (start 120 103.25) (end 120.7 105.5) (width 0.4) (layer "F.Cu") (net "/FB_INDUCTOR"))
 (segment (start 121.7 106.6) (end 121.7 106.2) (width 0.3) (layer "F.Cu") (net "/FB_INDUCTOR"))
 (via (at 116.5 104.9) (size 0.75) (drill 0.3) (layers "F.Cu" "B.Cu") (tenting (front yes) (back yes)) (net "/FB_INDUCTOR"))
 (via (at 121.7 106.2) (size 0.75) (drill 0.3) (layers "F.Cu" "B.Cu") (tenting (front yes) (back yes)) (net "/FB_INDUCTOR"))
 (via (at 120.7 105.5) (size 0.75) (drill 0.3) (layers "F.Cu" "B.Cu") (tenting (front yes) (back yes)) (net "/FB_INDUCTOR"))
 (segment (start 117.275 109) (end 116 107.725) (width 0.4) (layer "B.Cu") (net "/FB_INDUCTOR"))
 (segment (start 121.7 106.2) (end 122 105.3) (width 0.3) (layer "B.Cu") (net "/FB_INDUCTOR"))
 (segment (start 116 106) (end 117.3 106) (width 0.4) (layer "B.Cu") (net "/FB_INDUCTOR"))
 (segment (start 117.3 106) (end 117.3 105.1) (width 0.3) (layer "B.Cu") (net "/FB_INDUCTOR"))
 (segment (start 117.3 108.3) (end 120.3 111.3) (width 0.4) (layer "B.Cu") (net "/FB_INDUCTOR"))
 (segment (start 117.3 105.1) (end 116.5 104.9) (width 0.3) (layer "B.Cu") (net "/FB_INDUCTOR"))
 (segment (start 117.3 106) (end 117.3 108.3) (width 0.4) (layer "B.Cu") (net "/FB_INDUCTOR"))
 (segment (start 120.7 111.5) (end 121.2 112) (width 0.4) (layer "B.Cu") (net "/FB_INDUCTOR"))
 (segment (start 120.3 111.3) (end 121.2 112) (width 0.4) (layer "B.Cu") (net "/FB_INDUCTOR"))
 (segment (start 123.2 105.3) (end 123.2 106.335) (width 0.3) (layer "B.Cu") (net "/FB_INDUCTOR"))
 (segment (start 122 105.3) (end 123.2 105.3) (width 0.3) (layer "B.Cu") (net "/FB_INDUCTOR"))
 (segment (start 116 107.725) (end 116 106) (width 0.4) (layer "B.Cu") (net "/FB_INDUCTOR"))
 (segment (start 120.7 105.5) (end 120.7 111.5) (width 0.4) (layer "B.Cu") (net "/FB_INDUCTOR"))
 (segment (start 123.2 106.335) (end 124.725 106.335) (width 0.3) (layer "B.Cu") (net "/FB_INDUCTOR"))
 (segment (start 129 102) (end 127.15 101.3) (width 0.3) (layer "B.Cu") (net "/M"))
 (segment (start 126.8 104.2) (end 124.725 105.065) (width 0.3) (layer "B.Cu") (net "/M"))
 (segment (start 129 102) (end 126.8 102) (width 0.3) (layer "B.Cu") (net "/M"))
 (segment (start 126.8 102) (end 126.8 104.2) (width 0.3) (layer "B.Cu") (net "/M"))
 (segment (start 148.4 130.1) (end 145.7 128.4) (width 0.4) (layer "B.Cu") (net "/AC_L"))
 (segment (start 119.275 107.605) (end 119.275 103.795) (width 0.6) (layer "B.Cu") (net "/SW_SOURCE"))
 (segment (start 119.275 100.65) (end 119.275 103.795) (width 0.3) (layer "B.Cu") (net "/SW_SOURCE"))
 (segment (start 124.85 100.65) (end 119.275 100.65) (width 0.3) (layer "B.Cu") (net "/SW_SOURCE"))
 (segment (start 114.1 108.375) (end 114.1 106) (width 0.4) (layer "B.Cu") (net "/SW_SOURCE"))
 (segment (start 121 102) (end 119.275 103.025) (width 0.4) (layer "B.Cu") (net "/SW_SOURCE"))
 (segment (start 114.725 109) (end 114.1 108.375) (width 0.4) (layer "B.Cu") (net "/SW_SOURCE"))
 (segment (start 119.275 103.795) (end 114.1 103.795) (width 0.6) (layer "B.Cu") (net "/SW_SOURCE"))
 (segment (start 114.1 103.795) (end 114.1 106) (width 0.6) (layer "B.Cu") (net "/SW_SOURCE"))
 (segment (start 119.275 103.025) (end 119.275 103.795) (width 0.4) (layer "B.Cu") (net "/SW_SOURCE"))
 (segment (start 124.85 101.3) (end 124.85 100.65) (width 0.3) (layer "B.Cu") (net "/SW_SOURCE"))
 (segment (start 123 102) (end 124.725 103.025) (width 0.3) (layer "B.Cu") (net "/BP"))
 (segment (start 124.725 103.025) (end 124.725 103.795) (width 0.3) (layer "B.Cu") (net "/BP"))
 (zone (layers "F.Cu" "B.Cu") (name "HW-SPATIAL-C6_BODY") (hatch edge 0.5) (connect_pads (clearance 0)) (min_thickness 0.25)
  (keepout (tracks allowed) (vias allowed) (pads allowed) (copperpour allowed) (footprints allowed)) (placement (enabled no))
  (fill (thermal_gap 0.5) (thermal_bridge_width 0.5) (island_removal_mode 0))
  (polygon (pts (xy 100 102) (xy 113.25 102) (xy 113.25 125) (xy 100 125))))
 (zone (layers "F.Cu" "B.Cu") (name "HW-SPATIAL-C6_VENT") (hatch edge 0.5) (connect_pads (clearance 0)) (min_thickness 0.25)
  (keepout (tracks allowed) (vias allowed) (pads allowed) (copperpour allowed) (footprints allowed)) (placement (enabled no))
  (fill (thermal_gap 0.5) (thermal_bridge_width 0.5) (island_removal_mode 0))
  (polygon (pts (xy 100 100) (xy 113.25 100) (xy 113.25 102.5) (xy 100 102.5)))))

